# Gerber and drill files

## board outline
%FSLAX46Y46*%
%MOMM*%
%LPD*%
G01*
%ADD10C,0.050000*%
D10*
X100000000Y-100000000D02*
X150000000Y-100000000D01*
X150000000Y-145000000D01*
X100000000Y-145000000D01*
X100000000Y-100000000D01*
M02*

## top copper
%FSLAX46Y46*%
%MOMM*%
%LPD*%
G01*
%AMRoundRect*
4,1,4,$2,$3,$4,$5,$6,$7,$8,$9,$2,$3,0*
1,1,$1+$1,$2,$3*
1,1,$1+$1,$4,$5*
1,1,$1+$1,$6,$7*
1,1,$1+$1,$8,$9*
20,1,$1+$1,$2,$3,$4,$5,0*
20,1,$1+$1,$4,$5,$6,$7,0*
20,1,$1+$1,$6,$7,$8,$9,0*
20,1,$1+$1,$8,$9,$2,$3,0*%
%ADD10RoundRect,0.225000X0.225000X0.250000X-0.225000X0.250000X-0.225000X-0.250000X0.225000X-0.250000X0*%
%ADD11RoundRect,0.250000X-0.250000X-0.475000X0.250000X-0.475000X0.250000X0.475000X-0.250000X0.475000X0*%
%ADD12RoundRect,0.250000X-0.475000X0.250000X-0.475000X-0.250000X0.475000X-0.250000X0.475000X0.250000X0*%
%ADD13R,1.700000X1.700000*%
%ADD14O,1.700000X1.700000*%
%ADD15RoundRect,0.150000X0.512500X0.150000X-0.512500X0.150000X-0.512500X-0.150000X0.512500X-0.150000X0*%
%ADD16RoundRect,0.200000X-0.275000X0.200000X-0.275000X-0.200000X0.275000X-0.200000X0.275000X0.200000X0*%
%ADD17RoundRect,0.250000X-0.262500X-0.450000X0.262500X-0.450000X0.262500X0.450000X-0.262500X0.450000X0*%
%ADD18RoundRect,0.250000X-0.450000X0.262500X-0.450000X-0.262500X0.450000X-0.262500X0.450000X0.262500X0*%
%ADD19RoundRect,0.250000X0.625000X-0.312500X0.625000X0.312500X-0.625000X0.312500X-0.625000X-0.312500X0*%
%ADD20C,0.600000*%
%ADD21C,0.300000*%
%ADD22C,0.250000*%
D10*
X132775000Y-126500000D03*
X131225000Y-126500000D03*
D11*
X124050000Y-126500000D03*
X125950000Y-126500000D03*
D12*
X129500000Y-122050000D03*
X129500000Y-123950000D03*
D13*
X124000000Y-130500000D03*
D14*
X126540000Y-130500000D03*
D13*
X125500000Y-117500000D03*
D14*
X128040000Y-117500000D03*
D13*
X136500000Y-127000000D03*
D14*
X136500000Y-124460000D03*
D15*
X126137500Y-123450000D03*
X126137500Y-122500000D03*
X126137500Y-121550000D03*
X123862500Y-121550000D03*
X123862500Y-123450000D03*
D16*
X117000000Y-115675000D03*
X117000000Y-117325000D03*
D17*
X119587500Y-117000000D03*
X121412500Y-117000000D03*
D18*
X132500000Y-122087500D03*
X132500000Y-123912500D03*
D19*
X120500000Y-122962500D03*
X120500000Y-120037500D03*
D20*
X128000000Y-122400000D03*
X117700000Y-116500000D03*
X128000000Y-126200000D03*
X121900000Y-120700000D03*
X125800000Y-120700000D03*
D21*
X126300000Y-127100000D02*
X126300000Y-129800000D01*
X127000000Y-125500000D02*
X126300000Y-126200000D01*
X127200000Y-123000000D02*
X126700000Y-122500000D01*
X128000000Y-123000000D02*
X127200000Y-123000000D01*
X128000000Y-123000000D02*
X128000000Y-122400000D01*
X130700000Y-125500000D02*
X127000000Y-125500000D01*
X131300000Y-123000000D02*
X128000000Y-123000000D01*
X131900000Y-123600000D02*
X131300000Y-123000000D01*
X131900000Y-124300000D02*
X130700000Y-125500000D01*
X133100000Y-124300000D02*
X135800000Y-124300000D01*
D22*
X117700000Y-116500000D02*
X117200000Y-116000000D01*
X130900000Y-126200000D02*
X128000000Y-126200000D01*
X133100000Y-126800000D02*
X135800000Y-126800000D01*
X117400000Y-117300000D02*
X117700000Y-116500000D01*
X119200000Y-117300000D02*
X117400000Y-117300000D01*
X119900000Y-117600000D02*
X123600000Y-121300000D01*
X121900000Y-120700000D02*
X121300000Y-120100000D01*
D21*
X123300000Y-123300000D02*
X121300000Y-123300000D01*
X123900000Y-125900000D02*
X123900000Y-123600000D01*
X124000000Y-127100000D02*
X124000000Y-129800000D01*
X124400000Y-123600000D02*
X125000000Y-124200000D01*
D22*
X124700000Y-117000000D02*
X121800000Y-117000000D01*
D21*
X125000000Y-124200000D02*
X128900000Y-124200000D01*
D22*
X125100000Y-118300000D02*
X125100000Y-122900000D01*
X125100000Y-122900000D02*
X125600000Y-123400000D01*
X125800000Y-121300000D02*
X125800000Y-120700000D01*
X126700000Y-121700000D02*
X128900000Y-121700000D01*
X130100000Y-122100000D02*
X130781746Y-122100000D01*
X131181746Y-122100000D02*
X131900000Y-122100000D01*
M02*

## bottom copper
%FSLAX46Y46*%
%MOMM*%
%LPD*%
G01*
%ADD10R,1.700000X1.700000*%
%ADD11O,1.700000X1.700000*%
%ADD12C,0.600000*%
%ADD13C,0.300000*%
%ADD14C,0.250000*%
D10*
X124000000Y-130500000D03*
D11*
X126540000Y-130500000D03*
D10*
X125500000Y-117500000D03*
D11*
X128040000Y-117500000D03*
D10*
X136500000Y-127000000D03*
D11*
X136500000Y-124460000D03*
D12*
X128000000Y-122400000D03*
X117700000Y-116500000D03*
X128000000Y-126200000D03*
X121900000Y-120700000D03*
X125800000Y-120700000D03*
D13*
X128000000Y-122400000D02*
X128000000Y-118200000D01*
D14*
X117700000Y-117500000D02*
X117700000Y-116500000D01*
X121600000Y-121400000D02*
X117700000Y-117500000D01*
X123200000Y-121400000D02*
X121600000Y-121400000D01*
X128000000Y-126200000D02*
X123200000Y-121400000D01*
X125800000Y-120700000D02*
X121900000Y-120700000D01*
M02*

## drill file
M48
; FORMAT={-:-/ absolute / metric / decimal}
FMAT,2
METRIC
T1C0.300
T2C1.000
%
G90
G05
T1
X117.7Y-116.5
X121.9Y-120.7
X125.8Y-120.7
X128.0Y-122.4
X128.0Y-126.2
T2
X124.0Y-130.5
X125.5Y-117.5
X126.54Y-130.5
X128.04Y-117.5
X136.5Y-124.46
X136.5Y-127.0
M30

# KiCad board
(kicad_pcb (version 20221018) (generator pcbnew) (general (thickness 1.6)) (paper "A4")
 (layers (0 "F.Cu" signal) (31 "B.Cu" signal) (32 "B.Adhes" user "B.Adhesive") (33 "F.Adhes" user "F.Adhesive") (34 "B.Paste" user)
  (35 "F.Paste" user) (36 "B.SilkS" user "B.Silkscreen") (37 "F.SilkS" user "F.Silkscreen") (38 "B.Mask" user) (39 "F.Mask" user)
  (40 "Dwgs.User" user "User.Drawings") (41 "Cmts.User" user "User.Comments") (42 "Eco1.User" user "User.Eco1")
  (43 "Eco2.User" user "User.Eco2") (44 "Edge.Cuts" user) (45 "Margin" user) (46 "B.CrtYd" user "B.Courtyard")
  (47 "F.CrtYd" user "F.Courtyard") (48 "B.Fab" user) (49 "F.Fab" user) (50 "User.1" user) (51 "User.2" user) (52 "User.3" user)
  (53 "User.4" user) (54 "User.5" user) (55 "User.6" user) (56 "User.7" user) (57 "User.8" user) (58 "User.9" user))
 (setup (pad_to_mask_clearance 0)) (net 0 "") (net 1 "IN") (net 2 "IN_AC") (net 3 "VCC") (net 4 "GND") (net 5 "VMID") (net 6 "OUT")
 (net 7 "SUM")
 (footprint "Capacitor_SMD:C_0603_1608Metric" (layer "F.Cu") (at 132 126.5 180)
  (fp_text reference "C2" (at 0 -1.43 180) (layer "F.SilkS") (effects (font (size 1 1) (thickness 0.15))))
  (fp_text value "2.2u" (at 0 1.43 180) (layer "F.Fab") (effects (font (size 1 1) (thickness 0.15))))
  (pad "1" smd roundrect (at -0.775 0 180) (size 0.9 0.95) (layers "F.Cu" "F.Paste" "F.Mask") (roundrect_rratio 0.25) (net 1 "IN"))
  (pad "2" smd roundrect (at 0.775 0 180) (size 0.9 0.95) (layers "F.Cu" "F.Paste" "F.Mask") (roundrect_rratio 0.25) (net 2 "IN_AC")))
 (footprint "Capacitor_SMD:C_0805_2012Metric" (layer "F.Cu") (at 125 126.5)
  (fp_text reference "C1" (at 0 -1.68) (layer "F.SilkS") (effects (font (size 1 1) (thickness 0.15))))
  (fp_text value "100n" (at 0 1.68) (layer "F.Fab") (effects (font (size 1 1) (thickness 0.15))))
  (pad "1" smd roundrect (at -0.95 0) (size 1 1.45) (layers "F.Cu" "F.Paste" "F.Mask") (roundrect_rratio 0.25) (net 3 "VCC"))
  (pad "2" smd roundrect (at 0.95 0) (size 1 1.45) (layers "F.Cu" "F.Paste" "F.Mask") (roundrect_rratio 0.25) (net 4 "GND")))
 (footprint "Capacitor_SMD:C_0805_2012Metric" (layer "F.Cu") (at 129.5 123 -90)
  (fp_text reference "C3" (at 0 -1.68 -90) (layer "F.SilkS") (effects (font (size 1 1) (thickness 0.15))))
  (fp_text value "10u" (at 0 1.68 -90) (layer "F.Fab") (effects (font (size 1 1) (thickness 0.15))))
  (pad "1" smd roundrect (at -0.95 0 270) (size 1 1.45) (layers "F.Cu" "F.Paste" "F.Mask") (roundrect_rratio 0.25) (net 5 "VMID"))
  (pad "2" smd roundrect (at 0.95 0 270) (size 1 1.45) (layers "F.Cu" "F.Paste" "F.Mask") (roundrect_rratio 0.25) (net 3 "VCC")))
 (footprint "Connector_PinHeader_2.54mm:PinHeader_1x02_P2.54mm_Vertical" (layer "F.Cu") (at 124 130.5 90)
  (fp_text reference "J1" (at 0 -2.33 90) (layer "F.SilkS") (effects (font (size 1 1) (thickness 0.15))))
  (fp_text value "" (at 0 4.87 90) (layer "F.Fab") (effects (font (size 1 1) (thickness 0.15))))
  (pad "1" thru_hole rect (at 0 0 90) (size 1.7 1.7) (drill 1) (layers "*.Cu" "*.Mask") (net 3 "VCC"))
  (pad "2" thru_hole oval (at 0 2.54 90) (size 1.7 1.7) (drill 1) (layers "*.Cu" "*.Mask") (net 4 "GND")))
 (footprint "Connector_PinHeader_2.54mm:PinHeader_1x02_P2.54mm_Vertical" (layer "F.Cu") (at 125.5 117.5 90)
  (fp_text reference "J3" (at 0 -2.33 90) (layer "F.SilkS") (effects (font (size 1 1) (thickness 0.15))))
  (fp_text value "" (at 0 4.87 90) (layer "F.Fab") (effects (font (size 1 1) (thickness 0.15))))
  (pad "1" thru_hole rect (at 0 0 90) (size 1.7 1.7) (drill 1) (layers "*.Cu" "*.Mask") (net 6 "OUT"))
  (pad "2" thru_hole oval (at 0 2.54 90) (size 1.7 1.7) (drill 1) (layers "*.Cu" "*.Mask") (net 4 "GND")))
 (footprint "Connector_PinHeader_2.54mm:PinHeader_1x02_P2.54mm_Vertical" (layer "F.Cu") (at 136.5 127 180)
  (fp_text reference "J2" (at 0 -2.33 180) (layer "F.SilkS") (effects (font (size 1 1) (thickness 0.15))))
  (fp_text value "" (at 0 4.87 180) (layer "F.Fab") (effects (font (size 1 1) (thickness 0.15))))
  (pad "1" thru_hole rect (at 0 0 180) (size 1.7 1.7) (drill 1) (layers "*.Cu" "*.Mask") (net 1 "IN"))
  (pad "2" thru_hole oval (at 0 2.54 180) (size 1.7 1.7) (drill 1) (layers "*.Cu" "*.Mask") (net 4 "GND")))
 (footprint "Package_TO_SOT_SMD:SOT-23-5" (layer "F.Cu") (at 125 122.5 180)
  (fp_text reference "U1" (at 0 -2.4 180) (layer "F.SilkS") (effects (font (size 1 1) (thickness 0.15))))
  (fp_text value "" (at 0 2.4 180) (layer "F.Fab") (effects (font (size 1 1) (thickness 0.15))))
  (pad "1" smd roundrect (at -1.1375 -0.95 180) (size 1.325 0.6) (layers "F.Cu" "F.Paste" "F.Mask") (roundrect_rratio 0.25) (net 6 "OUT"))
  (pad "2" smd roundrect (at -1.1375 0 180) (size 1.325 0.6) (layers "F.Cu" "F.Paste" "F.Mask") (roundrect_rratio 0.25) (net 4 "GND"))
  (pad "3" smd roundrect (at -1.1375 0.95 180) (size 1.325 0.6) (layers "F.Cu" "F.Paste" "F.Mask") (roundrect_rratio 0.25) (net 5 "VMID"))
  (pad "4" smd roundrect (at 1.1375 0.95 180) (size 1.325 0.6) (layers "F.Cu" "F.Paste" "F.Mask") (roundrect_rratio 0.25) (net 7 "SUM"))
  (pad "5" smd roundrect (at 1.1375 -0.95 180) (size 1.325 0.6) (layers "F.Cu" "F.Paste" "F.Mask") (roundrect_rratio 0.25) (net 3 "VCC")))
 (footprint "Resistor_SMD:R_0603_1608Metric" (layer "F.Cu") (at 117 116.5 -90)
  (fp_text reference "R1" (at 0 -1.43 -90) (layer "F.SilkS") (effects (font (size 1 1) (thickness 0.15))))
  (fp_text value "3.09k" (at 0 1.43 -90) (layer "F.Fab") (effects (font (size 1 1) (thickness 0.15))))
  (pad "1" smd roundrect (at -0.825 0 270) (size 0.8 0.95) (layers "F.Cu" "F.Paste" "F.Mask") (roundrect_rratio 0.25) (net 2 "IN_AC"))
  (pad "2" smd roundrect (at 0.825 0 270) (size 0.8 0.95) (layers "F.Cu" "F.Paste" "F.Mask") (roundrect_rratio 0.25) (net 7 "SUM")))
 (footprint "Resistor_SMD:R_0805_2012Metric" (layer "F.Cu") (at 120.5 117)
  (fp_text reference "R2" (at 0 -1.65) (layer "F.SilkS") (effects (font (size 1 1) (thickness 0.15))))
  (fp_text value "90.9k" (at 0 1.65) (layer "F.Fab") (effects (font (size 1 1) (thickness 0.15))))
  (pad "1" smd roundrect (at -0.9125 0) (size 1.025 1.4) (layers "F.Cu" "F.Paste" "F.Mask") (roundrect_rratio 0.243902) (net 7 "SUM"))
  (pad "2" smd roundrect (at 0.9125 0) (size 1.025 1.4) (layers "F.Cu" "F.Paste" "F.Mask") (roundrect_rratio 0.243902) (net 6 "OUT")))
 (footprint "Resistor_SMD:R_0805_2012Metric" (layer "F.Cu") (at 132.5 123 -90)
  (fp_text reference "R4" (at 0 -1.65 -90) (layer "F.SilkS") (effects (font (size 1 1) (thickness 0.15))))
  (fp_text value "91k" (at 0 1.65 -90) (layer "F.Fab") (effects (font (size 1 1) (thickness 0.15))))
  (pad "1" smd roundrect (at -0.9125 0 270) (size 1.025 1.4) (layers "F.Cu" "F.Paste" "F.Mask") (roundrect_rratio 0.243902) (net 5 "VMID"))
  (pad "2" smd roundrect (at 0.9125 0 270) (size 1.025 1.4) (layers "F.Cu" "F.Paste" "F.Mask") (roundrect_rratio 0.243902) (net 4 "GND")))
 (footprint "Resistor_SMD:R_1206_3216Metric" (layer "F.Cu") (at 120.5 121.5 90)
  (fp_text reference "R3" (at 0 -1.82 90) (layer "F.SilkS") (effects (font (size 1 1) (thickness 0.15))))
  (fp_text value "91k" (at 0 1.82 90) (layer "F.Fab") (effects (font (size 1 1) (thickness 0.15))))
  (pad "1" smd roundrect (at -1.4625 0 90) (size 1.125 1.75) (layers "F.Cu" "F.Paste" "F.Mask") (roundrect_rratio 0.222222) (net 3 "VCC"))
  (pad "2" smd roundrect (at 1.4625 0 90) (size 1.125 1.75) (layers "F.Cu" "F.Paste" "F.Mask") (roundrect_rratio 0.222222) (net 5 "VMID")))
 (gr_rect (start 100 100) (end 150 145) (stroke (width 0.05) (type default)) (fill none) (layer "Edge.Cuts"))
 (segment (start 126.3 127.1) (end 126.3 129.8) (width 0.3) (layer "F.Cu") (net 4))
 (segment (start 127 125.5) (end 126.3 126.2) (width 0.3) (layer "F.Cu") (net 4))
 (segment (start 127.2 123) (end 126.7 122.5) (width 0.3) (layer "F.Cu") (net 4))
 (segment (start 128 123) (end 127.2 123) (width 0.3) (layer "F.Cu") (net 4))
 (segment (start 128 123) (end 128 122.4) (width 0.3) (layer "F.Cu") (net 4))
 (segment (start 130.7 125.5) (end 127 125.5) (width 0.3) (layer "F.Cu") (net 4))
 (segment (start 131.3 123) (end 128 123) (width 0.3) (layer "F.Cu") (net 4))
 (segment (start 131.9 123.6) (end 131.3 123) (width 0.3) (layer "F.Cu") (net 4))
 (segment (start 131.9 124.3) (end 130.7 125.5) (width 0.3) (layer "F.Cu") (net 4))
 (segment (start 133.1 124.3) (end 135.8 124.3) (width 0.3) (layer "F.Cu") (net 4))
 (via (at 128 122.4) (size 0.6) (drill 0.3) (layers "F.Cu" "B.Cu") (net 4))
 (segment (start 117.7 116.5) (end 117.2 116) (width 0.25) (layer "F.Cu") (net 2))
 (segment (start 128 122.4) (end 128 118.2) (width 0.3) (layer "B.Cu") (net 4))
 (segment (start 130.9 126.2) (end 128 126.2) (width 0.25) (layer "F.Cu") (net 2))
 (segment (start 133.1 126.8) (end 135.8 126.8) (width 0.25) (layer "F.Cu") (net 1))
 (via (at 117.7 116.5) (size 0.6) (drill 0.3) (layers "F.Cu" "B.Cu") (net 2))
 (via (at 128 126.2) (size 0.6) (drill 0.3) (layers "F.Cu" "B.Cu") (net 2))
 (segment (start 117.4 117.3) (end 117.7 116.5) (width 0.25) (layer "F.Cu") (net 7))
 (segment (start 117.7 117.5) (end 117.7 116.5) (width 0.25) (layer "B.Cu") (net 2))
 (segment (start 119.2 117.3) (end 117.4 117.3) (width 0.25) (layer "F.Cu") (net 7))
 (segment (start 119.9 117.6) (end 123.6 121.3) (width 0.25) (layer "F.Cu") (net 7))
 (segment (start 121.6 121.4) (end 117.7 117.5) (width 0.25) (layer "B.Cu") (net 2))
 (segment (start 121.9 120.7) (end 121.3 120.1) (width 0.25) (layer "F.Cu") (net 5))
 (segment (start 123.2 121.4) (end 121.6 121.4) (width 0.25) (layer "B.Cu") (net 2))
 (segment (start 123.3 123.3) (end 121.3 123.3) (width 0.3) (layer "F.Cu") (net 3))
 (segment (start 123.9 125.9) (end 123.9 123.6) (width 0.3) (layer "F.Cu") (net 3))
 (segment (start 124 127.1) (end 124 129.8) (width 0.3) (layer "F.Cu") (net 3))
 (segment (start 124.4 123.6) (end 125 124.2) (width 0.3) (layer "F.Cu") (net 3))
 (segment (start 124.7 117) (end 121.8 117) (width 0.25) (layer "F.Cu") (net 6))
 (segment (start 125 124.2) (end 128.9 124.2) (width 0.3) (layer "F.Cu") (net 3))
 (segment (start 125.1 118.3) (end 125.1 122.9) (width 0.25) (layer "F.Cu") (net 6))
 (segment (start 125.1 122.9) (end 125.6 123.4) (width 0.25) (layer "F.Cu") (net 6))
 (segment (start 125.8 121.3) (end 125.8 120.7) (width 0.25) (layer "F.Cu") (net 5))
 (segment (start 126.7 121.7) (end 128.9 121.7) (width 0.25) (layer "F.Cu") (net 5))
 (segment (start 128 126.2) (end 123.2 121.4) (width 0.25) (layer "B.Cu") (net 2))
 (segment (start 130.1 122.1) (end 130.781746 122.1) (width 0.25) (layer "F.Cu") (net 5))
 (segment (start 131.181746 122.1) (end 131.9 122.1) (width 0.25) (layer "F.Cu") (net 5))
 (via (at 121.9 120.7) (size 0.6) (drill 0.3) (layers "F.Cu" "B.Cu") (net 5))
 (via (at 125.8 120.7) (size 0.6) (drill 0.3) (layers "F.Cu" "B.Cu") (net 5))
 (segment (start 125.8 120.7) (end 121.9 120.7) (width 0.25) (layer "B.Cu") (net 5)))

